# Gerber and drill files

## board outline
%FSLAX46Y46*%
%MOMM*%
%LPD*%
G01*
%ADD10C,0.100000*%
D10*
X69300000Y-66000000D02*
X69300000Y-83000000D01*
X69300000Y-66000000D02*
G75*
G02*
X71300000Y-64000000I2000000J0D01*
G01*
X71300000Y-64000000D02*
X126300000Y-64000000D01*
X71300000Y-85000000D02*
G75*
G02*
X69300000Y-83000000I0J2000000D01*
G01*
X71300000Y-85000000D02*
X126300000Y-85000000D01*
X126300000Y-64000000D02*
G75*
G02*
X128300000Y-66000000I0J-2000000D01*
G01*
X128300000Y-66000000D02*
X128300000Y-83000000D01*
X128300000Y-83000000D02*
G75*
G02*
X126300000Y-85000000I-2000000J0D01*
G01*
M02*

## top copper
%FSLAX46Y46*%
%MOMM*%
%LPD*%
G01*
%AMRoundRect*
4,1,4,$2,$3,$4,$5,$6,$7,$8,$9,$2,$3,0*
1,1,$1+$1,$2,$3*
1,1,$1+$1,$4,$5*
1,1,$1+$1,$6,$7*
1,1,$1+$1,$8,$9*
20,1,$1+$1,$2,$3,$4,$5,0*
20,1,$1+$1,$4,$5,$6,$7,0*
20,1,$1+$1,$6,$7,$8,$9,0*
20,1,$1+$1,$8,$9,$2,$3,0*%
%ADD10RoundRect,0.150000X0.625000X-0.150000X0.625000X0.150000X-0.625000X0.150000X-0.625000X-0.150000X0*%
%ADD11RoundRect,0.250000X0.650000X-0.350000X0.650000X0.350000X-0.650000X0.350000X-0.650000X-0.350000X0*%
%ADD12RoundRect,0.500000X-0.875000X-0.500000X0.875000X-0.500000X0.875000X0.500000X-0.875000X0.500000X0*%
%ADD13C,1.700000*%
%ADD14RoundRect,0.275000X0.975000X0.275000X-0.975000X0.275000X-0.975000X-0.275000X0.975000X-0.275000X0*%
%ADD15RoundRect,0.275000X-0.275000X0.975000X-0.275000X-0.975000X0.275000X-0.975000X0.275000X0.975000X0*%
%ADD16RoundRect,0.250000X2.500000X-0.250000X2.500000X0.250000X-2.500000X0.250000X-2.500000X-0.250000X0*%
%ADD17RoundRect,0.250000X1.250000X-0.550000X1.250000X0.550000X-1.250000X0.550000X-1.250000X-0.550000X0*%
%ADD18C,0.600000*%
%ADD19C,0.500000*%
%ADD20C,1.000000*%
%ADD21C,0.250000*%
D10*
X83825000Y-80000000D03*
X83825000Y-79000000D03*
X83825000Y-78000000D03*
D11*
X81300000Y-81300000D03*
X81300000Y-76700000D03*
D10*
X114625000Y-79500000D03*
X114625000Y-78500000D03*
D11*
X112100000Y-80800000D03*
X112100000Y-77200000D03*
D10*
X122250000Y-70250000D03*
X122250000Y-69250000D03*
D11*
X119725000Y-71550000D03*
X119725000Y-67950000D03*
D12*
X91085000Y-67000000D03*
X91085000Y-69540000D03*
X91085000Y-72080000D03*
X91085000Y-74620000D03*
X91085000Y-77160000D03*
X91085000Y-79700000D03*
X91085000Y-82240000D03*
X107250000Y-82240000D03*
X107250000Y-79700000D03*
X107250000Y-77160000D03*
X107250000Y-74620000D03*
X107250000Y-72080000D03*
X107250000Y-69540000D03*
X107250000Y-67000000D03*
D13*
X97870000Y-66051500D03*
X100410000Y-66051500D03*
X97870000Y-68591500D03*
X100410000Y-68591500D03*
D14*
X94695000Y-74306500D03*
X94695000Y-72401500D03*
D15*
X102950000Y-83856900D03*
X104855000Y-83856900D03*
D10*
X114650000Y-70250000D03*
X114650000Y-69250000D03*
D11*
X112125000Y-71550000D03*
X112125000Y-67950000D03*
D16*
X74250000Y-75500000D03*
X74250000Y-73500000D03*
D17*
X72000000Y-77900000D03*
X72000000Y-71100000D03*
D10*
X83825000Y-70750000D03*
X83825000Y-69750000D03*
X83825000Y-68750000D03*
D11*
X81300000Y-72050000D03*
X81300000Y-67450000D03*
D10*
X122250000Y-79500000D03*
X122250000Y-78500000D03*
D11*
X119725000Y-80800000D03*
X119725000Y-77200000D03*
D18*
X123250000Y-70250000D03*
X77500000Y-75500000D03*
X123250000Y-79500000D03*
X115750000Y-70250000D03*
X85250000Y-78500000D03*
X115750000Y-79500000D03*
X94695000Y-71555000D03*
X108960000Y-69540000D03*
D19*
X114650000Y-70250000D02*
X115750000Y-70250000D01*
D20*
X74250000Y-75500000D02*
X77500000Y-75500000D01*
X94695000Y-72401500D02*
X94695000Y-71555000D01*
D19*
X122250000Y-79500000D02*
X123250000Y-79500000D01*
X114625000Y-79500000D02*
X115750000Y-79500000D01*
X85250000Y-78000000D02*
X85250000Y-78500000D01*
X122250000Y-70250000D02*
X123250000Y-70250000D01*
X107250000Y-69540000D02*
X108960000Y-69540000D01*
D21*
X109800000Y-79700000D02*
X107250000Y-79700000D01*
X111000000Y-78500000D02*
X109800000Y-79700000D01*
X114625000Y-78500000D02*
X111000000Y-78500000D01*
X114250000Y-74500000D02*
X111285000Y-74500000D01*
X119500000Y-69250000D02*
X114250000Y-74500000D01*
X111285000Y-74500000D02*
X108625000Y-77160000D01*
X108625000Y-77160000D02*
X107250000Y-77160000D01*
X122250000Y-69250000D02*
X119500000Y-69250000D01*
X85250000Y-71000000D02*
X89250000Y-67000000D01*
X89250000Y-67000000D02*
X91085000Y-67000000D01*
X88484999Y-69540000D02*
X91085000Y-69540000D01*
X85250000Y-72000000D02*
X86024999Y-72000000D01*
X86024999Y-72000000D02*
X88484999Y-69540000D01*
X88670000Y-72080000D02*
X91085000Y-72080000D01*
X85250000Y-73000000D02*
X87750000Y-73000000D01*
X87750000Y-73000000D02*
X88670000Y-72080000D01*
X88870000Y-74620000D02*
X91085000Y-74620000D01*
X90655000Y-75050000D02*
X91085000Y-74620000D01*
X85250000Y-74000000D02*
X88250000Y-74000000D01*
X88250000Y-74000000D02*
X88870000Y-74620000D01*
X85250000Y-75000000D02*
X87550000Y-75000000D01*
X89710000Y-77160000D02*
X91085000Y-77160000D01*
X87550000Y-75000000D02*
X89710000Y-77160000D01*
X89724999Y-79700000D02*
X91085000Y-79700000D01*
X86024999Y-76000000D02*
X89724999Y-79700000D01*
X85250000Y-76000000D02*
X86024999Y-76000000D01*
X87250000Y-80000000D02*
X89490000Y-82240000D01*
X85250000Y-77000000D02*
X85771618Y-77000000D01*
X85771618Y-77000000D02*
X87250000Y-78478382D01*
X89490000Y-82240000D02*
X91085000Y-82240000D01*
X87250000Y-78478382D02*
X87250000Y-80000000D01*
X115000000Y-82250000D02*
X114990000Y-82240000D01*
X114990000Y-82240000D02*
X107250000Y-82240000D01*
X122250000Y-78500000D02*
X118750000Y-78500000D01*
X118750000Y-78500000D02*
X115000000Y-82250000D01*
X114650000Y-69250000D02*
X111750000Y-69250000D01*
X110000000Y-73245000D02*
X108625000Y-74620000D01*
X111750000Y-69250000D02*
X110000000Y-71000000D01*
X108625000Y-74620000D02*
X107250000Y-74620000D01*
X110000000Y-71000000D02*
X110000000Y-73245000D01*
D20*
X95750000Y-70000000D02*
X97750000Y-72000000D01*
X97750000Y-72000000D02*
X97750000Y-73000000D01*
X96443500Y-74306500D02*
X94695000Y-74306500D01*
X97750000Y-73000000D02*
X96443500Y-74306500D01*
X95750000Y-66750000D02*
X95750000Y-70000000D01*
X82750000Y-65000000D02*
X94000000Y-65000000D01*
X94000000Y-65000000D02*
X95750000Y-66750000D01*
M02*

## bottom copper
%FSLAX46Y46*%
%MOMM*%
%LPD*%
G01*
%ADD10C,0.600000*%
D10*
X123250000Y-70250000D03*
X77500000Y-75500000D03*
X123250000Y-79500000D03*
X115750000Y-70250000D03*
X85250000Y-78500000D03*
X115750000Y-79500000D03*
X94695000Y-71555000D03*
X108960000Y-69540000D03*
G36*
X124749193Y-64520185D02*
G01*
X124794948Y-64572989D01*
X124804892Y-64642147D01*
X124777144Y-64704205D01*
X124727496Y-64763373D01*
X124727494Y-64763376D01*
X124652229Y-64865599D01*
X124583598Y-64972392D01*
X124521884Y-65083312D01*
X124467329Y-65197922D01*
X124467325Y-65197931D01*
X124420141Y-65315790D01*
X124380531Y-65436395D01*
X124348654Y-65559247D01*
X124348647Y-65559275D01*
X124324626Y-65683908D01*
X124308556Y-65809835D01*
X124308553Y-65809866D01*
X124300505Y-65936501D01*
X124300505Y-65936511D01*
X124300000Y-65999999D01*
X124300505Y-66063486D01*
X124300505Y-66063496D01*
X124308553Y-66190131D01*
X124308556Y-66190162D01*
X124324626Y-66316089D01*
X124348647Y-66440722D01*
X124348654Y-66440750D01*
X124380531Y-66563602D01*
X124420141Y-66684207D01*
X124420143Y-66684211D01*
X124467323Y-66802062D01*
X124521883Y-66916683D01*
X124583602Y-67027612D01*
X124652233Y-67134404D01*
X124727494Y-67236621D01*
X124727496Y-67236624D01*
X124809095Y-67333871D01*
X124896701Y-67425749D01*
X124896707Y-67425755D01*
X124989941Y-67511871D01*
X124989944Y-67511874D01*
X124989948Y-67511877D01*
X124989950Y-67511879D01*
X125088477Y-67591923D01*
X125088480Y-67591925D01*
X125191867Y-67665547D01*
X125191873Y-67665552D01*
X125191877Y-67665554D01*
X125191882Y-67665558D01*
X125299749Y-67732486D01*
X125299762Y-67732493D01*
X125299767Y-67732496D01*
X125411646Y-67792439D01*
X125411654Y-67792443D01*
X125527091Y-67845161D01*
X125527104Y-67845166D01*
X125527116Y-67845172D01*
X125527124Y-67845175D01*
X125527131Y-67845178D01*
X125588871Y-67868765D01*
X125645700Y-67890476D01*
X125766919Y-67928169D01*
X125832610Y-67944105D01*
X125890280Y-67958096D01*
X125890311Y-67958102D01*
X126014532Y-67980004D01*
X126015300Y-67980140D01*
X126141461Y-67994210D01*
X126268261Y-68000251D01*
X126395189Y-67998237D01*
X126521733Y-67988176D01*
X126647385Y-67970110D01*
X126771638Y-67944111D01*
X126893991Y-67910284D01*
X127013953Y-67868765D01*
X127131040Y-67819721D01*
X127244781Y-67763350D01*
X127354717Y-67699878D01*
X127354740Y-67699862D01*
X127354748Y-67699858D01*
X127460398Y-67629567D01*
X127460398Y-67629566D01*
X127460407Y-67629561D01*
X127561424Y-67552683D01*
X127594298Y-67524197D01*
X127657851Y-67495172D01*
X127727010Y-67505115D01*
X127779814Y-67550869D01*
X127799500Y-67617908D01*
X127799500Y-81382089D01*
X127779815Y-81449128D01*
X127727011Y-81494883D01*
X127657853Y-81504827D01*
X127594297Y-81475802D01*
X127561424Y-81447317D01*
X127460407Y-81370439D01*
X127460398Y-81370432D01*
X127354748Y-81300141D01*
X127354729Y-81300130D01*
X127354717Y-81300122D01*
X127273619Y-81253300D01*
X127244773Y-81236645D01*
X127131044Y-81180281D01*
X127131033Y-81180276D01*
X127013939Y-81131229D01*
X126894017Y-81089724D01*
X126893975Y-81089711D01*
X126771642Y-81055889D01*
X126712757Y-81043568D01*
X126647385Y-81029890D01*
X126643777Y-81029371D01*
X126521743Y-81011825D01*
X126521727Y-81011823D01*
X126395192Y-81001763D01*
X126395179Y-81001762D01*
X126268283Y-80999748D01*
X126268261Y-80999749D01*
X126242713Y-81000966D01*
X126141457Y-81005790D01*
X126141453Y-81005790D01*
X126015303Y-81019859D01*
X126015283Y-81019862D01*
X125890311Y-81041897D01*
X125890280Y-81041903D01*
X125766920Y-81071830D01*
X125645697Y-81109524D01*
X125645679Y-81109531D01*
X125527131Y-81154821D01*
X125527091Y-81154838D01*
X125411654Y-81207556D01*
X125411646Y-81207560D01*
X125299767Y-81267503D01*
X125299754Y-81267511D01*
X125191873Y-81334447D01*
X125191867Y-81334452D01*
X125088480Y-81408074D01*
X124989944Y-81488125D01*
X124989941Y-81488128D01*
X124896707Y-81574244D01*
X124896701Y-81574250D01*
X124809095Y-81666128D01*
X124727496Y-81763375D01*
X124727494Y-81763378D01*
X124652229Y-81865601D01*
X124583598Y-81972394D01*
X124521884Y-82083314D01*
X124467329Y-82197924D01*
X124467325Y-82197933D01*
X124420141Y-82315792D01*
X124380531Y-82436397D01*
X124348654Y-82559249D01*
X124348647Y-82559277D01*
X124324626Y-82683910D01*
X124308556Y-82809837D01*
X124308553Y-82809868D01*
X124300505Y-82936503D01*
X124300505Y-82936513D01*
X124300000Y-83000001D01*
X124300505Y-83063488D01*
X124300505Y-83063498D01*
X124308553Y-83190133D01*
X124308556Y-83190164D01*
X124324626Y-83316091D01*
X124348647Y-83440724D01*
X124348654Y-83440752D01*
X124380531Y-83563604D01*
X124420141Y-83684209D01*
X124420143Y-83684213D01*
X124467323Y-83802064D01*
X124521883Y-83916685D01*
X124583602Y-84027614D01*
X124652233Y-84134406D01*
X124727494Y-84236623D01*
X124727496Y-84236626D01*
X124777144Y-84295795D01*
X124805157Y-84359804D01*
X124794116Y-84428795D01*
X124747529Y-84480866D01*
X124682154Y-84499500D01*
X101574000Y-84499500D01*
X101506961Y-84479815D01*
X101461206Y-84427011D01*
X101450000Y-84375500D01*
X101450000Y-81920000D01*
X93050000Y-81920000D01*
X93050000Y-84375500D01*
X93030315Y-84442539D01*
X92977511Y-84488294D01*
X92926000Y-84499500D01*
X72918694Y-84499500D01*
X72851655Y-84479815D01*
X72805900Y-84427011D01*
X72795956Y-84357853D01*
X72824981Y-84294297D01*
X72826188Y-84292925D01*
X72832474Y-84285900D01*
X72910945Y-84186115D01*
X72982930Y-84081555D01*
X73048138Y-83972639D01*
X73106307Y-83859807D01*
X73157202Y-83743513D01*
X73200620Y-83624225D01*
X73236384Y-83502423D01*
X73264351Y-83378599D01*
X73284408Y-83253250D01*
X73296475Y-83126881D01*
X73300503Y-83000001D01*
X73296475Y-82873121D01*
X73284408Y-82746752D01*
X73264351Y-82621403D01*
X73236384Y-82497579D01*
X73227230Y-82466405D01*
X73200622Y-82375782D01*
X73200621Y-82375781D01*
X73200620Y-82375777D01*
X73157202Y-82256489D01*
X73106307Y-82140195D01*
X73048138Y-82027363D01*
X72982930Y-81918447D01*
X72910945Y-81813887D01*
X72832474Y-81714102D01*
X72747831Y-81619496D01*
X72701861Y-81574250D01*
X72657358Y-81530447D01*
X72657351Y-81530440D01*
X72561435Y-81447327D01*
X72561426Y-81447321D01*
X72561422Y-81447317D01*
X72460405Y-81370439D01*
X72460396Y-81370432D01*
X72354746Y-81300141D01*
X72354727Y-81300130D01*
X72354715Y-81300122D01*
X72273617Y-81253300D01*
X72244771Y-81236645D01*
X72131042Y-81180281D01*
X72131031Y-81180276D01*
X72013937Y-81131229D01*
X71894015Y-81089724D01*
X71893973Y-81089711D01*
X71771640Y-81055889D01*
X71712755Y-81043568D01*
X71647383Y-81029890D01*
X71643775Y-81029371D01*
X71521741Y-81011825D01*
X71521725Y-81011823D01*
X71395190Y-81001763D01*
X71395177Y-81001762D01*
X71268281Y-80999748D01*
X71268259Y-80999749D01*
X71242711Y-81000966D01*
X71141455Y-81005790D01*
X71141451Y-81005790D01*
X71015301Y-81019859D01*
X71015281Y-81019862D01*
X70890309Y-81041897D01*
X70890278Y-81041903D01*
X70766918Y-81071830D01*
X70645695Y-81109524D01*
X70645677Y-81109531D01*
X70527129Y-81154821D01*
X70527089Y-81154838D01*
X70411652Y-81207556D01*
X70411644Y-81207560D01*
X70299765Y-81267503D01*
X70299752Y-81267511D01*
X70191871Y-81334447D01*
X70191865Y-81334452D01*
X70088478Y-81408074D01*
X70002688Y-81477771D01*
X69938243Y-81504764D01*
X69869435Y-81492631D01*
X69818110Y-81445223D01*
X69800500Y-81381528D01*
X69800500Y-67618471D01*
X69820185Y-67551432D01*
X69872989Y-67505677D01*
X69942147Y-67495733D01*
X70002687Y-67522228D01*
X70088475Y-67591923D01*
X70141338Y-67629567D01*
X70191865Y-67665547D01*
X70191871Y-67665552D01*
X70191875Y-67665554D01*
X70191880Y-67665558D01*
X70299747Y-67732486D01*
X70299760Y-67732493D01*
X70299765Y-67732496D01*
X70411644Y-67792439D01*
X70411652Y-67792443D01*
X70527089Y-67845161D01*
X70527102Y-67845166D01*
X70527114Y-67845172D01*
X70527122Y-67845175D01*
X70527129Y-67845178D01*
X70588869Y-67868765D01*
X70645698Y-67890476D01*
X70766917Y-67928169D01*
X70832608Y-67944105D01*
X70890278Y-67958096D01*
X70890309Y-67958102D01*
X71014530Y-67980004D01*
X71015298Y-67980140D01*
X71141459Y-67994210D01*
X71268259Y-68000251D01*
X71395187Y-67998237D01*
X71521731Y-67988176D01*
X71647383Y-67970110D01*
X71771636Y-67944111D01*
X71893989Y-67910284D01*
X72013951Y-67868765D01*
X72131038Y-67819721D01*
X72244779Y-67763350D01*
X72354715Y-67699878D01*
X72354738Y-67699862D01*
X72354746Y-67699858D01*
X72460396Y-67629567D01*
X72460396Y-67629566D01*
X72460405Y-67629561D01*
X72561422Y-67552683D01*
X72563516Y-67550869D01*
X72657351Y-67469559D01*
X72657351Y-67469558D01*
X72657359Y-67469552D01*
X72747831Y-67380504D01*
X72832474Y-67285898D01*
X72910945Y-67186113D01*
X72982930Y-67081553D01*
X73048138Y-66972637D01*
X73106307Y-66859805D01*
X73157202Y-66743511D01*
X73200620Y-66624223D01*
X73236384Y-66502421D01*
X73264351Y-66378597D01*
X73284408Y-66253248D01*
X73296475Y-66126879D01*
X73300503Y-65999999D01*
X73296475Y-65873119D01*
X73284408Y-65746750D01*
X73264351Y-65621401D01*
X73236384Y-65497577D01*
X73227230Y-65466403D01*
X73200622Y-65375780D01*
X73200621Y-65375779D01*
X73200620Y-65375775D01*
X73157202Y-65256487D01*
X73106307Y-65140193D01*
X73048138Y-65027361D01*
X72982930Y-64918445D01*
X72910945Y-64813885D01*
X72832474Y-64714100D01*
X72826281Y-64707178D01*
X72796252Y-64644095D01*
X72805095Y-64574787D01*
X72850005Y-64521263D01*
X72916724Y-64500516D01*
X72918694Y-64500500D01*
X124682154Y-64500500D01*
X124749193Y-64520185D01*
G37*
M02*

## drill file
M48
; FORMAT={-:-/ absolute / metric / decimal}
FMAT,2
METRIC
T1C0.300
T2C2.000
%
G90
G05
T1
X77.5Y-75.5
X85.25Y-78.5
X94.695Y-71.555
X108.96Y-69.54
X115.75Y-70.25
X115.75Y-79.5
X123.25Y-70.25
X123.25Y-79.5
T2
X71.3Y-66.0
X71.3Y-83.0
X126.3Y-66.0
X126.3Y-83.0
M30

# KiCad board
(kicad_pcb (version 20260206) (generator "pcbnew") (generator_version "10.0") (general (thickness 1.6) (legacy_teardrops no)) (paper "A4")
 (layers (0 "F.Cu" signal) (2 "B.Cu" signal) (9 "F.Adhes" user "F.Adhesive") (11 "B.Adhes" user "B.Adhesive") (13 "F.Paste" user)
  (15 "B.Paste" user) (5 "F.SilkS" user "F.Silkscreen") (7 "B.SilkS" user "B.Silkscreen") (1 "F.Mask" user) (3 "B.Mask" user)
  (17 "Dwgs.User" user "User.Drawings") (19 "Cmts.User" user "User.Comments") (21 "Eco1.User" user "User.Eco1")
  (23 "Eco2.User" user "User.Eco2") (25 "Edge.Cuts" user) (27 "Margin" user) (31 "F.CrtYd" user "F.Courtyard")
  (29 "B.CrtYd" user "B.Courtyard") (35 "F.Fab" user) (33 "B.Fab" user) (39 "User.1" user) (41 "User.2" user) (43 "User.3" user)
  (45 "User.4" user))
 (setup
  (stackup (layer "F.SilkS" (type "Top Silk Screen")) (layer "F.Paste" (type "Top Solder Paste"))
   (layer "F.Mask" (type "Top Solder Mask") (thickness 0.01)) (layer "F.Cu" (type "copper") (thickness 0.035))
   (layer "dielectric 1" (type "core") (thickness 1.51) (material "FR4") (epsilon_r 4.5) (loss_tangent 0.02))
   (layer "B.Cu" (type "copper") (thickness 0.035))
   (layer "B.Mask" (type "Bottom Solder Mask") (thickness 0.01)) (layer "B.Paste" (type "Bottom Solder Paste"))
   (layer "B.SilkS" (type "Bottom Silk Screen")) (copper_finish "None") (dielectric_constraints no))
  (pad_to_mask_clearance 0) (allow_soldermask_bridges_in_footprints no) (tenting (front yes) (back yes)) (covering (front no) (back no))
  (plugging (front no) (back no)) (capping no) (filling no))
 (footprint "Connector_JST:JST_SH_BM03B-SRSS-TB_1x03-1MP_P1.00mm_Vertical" (layer "F.Cu") (at 82.5 79 90)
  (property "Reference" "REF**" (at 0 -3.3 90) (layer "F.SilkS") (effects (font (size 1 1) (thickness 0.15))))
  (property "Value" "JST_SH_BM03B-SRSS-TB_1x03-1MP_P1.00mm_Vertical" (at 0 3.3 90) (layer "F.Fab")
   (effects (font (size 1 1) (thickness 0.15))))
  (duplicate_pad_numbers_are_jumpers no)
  (pad "1" smd roundrect (at -1 1.325 90) (size 0.6 1.55) (layers "F.Cu" "F.Mask" "F.Paste") (roundrect_rratio 0.25))
  (pad "2" smd roundrect (at 0 1.325 90) (size 0.6 1.55) (layers "F.Cu" "F.Mask" "F.Paste") (roundrect_rratio 0.25))
  (pad "3" smd roundrect (at 1 1.325 90) (size 0.6 1.55) (layers "F.Cu" "F.Mask" "F.Paste") (roundrect_rratio 0.25))
  (pad "MP" smd roundrect (at -2.3 -1.2 90) (size 1.2 1.8) (layers "F.Cu" "F.Mask" "F.Paste") (roundrect_rratio 0.208333))
  (pad "MP" smd roundrect (at 2.3 -1.2 90) (size 1.2 1.8) (layers "F.Cu" "F.Mask" "F.Paste") (roundrect_rratio 0.208333)))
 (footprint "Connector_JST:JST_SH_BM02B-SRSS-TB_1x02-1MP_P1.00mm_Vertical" (layer "F.Cu") (at 113.3 79 90)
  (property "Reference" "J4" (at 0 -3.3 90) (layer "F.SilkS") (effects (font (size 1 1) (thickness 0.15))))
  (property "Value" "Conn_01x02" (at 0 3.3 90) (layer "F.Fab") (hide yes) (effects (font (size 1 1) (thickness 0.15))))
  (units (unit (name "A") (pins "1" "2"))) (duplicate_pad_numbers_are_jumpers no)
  (pad "1" smd roundrect (at -0.5 1.325 90) (size 0.6 1.55) (layers "F.Cu" "F.Mask" "F.Paste") (roundrect_rratio 0.25) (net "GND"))
  (pad "2" smd roundrect (at 0.5 1.325 90) (size 0.6 1.55) (layers "F.Cu" "F.Mask" "F.Paste") (roundrect_rratio 0.25) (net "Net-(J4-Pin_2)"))
  (pad "MP" smd roundrect (at -1.8 -1.2 90) (size 1.2 1.8) (layers "F.Cu" "F.Mask" "F.Paste") (roundrect_rratio 0.208333))
  (pad "MP" smd roundrect (at 1.8 -1.2 90) (size 1.2 1.8) (layers "F.Cu" "F.Mask" "F.Paste") (roundrect_rratio 0.208333)))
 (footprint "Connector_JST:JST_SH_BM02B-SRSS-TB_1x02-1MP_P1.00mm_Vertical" (layer "F.Cu") (at 120.925 69.75 90)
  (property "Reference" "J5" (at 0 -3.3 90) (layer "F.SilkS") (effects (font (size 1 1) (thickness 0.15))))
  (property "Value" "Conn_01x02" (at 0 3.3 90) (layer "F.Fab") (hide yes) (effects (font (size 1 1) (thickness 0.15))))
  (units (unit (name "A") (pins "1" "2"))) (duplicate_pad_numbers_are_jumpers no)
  (pad "1" smd roundrect (at -0.5 1.325 90) (size 0.6 1.55) (layers "F.Cu" "F.Mask" "F.Paste") (roundrect_rratio 0.25) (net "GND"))
  (pad "2" smd roundrect (at 0.5 1.325 90) (size 0.6 1.55) (layers "F.Cu" "F.Mask" "F.Paste") (roundrect_rratio 0.25) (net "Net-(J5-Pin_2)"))
  (pad "MP" smd roundrect (at -1.8 -1.2 90) (size 1.2 1.8) (layers "F.Cu" "F.Mask" "F.Paste") (roundrect_rratio 0.208333))
  (pad "MP" smd roundrect (at 1.8 -1.2 90) (size 1.2 1.8) (layers "F.Cu" "F.Mask" "F.Paste") (roundrect_rratio 0.208333)))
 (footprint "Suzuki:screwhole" (layer "F.Cu") (at 126.300001 65.999999)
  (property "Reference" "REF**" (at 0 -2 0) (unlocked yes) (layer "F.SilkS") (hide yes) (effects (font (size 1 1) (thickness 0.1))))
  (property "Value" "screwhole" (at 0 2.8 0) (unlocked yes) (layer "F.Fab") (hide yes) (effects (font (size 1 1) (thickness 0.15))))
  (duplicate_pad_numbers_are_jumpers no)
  (pad "" np_thru_hole circle (at 0 0) (size 2 2) (drill 2) (layers "*.Cu" "*.Mask"))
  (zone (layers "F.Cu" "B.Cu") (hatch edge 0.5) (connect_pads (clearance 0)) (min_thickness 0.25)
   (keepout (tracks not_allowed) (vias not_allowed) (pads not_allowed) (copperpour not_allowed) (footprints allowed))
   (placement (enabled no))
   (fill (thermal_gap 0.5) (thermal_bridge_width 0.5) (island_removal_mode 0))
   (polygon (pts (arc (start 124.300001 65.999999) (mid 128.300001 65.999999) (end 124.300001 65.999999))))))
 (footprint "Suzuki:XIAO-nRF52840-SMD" (layer "F.Cu") (at 90.25 85.12)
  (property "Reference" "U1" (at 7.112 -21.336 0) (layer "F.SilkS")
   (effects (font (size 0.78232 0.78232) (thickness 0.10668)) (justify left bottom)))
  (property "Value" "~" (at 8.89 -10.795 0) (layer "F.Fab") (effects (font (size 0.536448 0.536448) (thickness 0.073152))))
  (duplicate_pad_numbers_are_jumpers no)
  (pad "1" smd roundrect (at 0.835 -18.12) (size 2.75 2) (layers "F.Cu" "F.Mask" "F.Paste") (roundrect_rratio 0.25) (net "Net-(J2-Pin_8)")
   (solder_mask_margin 0.0508) (thermal_bridge_angle 45))
  (pad "2" smd roundrect (at 0.835 -15.58) (size 2.75 2) (layers "F.Cu" "F.Mask" "F.Paste") (roundrect_rratio 0.25) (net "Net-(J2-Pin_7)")
   (solder_mask_margin 0.0508) (thermal_bridge_angle 45))
  (pad "3" smd roundrect (at 0.835 -13.04) (size 2.75 2) (layers "F.Cu" "F.Mask" "F.Paste") (roundrect_rratio 0.25) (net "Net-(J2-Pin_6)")
   (solder_mask_margin 0.0508) (thermal_bridge_angle 45))
  (pad "4" smd roundrect (at 0.835 -10.5) (size 2.75 2) (layers "F.Cu" "F.Mask" "F.Paste") (roundrect_rratio 0.25) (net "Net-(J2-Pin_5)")
   (solder_mask_margin 0.0508) (thermal_bridge_angle 45))
  (pad "5" smd roundrect (at 0.835 -7.96) (size 2.75 2) (layers "F.Cu" "F.Mask" "F.Paste") (roundrect_rratio 0.25) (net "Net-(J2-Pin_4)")
   (solder_mask_margin 0.0508) (thermal_bridge_angle 45))
  (pad "6" smd roundrect (at 0.835 -5.42) (size 2.75 2) (layers "F.Cu" "F.Mask" "F.Paste") (roundrect_rratio 0.25) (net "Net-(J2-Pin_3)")
   (solder_mask_margin 0.0508) (thermal_bridge_angle 45))
  (pad "7" smd roundrect (at 0.835 -2.88) (size 2.75 2) (layers "F.Cu" "F.Mask" "F.Paste") (roundrect_rratio 0.25) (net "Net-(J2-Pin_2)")
   (solder_mask_margin 0.0508) (thermal_bridge_angle 45))
  (pad "8" smd roundrect (at 17 -2.88) (size 2.75 2) (layers "F.Cu" "F.Mask" "F.Paste") (roundrect_rratio 0.25) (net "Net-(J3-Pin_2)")
   (solder_mask_margin 0.0508) (thermal_bridge_angle 45))
  (pad "9" smd roundrect (at 17 -5.42) (size 2.75 2) (layers "F.Cu" "F.Mask" "F.Paste") (roundrect_rratio 0.25) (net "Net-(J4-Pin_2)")
   (solder_mask_margin 0.0508) (thermal_bridge_angle 45))
  (pad "10" smd roundrect (at 17 -7.96) (size 2.75 2) (layers "F.Cu" "F.Mask" "F.Paste") (roundrect_rratio 0.25) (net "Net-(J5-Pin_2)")
   (solder_mask_margin 0.0508) (thermal_bridge_angle 45))
  (pad "11" smd roundrect (at 17 -10.5) (size 2.75 2) (layers "F.Cu" "F.Mask" "F.Paste") (roundrect_rratio 0.25) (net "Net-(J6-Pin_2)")
   (solder_mask_margin 0.0508) (thermal_bridge_angle 45))
  (pad "12" smd roundrect (at 17 -13.04) (size 2.75 2) (layers "F.Cu" "F.Mask" "F.Paste") (roundrect_rratio 0.25)
   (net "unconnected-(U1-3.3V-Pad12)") (solder_mask_margin 0.0508) (thermal_bridge_angle 45))
  (pad "13" smd roundrect (at 17 -15.58) (size 2.75 2) (layers "F.Cu" "F.Mask" "F.Paste") (roundrect_rratio 0.25) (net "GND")
   (solder_mask_margin 0.0508) (thermal_bridge_angle 45))
  (pad "14" smd roundrect (at 17 -18.12) (size 2.75 2) (layers "F.Cu" "F.Mask" "F.Paste") (roundrect_rratio 0.25)
   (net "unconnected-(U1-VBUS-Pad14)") (solder_mask_margin 0.0508) (thermal_bridge_angle 45))
  (pad "15" smd circle (at 7.62 -19.0685) (size 1.7 1.7) (layers "F.Cu" "F.Mask" "F.Paste"))
  (pad "16" smd circle (at 10.16 -19.0685) (size 1.7 1.7) (layers "F.Cu" "F.Mask" "F.Paste"))
  (pad "17" smd circle (at 7.62 -16.5285) (size 1.7 1.7) (layers "F.Cu" "F.Mask" "F.Paste"))
  (pad "18" smd circle (at 10.16 -16.5285) (size 1.7 1.7) (layers "F.Cu" "F.Mask" "F.Paste"))
  (pad "19" smd roundrect (at 4.445 -10.8135 180) (size 2.5 1.1) (layers "F.Cu" "F.Mask" "F.Paste") (roundrect_rratio 0.25)
   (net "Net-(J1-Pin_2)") (thermal_bridge_angle 45))
  (pad "20" smd roundrect (at 4.445 -12.7185 180) (size 2.5 1.1) (layers "F.Cu" "F.Mask" "F.Paste") (roundrect_rratio 0.25) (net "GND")
   (thermal_bridge_angle 45))
  (pad "21" smd roundrect (at 12.7 -1.2631 270) (size 2.5 1.1) (layers "F.Cu" "F.Mask" "F.Paste") (roundrect_rratio 0.25)
   (thermal_bridge_angle 45))
  (pad "22" smd roundrect (at 14.605 -1.2631 270) (size 2.5 1.1) (layers "F.Cu" "F.Mask" "F.Paste") (roundrect_rratio 0.25)
   (thermal_bridge_angle 45))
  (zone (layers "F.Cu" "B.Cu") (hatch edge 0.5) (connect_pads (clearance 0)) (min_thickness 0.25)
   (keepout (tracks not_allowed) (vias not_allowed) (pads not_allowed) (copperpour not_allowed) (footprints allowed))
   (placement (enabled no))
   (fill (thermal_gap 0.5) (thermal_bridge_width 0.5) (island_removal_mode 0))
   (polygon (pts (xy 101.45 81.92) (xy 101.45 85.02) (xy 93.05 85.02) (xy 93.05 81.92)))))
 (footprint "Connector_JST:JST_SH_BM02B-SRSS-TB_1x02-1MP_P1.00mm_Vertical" (layer "F.Cu") (at 113.325 69.75 90)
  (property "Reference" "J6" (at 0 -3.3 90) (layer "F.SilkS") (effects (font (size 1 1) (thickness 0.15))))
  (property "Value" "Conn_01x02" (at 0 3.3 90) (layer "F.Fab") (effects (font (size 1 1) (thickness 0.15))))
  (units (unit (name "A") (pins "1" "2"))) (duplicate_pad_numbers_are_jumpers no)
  (pad "1" smd roundrect (at -0.5 1.325 90) (size 0.6 1.55) (layers "F.Cu" "F.Mask" "F.Paste") (roundrect_rratio 0.25) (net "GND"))
  (pad "2" smd roundrect (at 0.5 1.325 90) (size 0.6 1.55) (layers "F.Cu" "F.Mask" "F.Paste") (roundrect_rratio 0.25) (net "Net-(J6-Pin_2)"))
  (pad "MP" smd roundrect (at -1.8 -1.2 90) (size 1.2 1.8) (layers "F.Cu" "F.Mask" "F.Paste") (roundrect_rratio 0.208333))
  (pad "MP" smd roundrect (at 1.8 -1.2 90) (size 1.2 1.8) (layers "F.Cu" "F.Mask" "F.Paste") (roundrect_rratio 0.208333)))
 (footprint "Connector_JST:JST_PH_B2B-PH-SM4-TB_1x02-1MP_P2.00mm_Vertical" (layer "F.Cu") (at 73.75 74.5 90)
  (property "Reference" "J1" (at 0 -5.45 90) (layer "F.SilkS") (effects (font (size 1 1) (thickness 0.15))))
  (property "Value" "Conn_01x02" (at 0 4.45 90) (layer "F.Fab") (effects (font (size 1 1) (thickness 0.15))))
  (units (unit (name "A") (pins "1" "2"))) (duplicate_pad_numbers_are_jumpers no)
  (pad "1" smd roundrect (at -1 0.5 90) (size 1 5.5) (layers "F.Cu" "F.Mask" "F.Paste") (roundrect_rratio 0.25) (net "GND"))
  (pad "2" smd roundrect (at 1 0.5 90) (size 1 5.5) (layers "F.Cu" "F.Mask" "F.Paste") (roundrect_rratio 0.25) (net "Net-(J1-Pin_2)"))
  (pad "MP" smd roundrect (at -3.4 -1.75 90) (size 1.6 3) (layers "F.Cu" "F.Mask" "F.Paste") (roundrect_rratio 0.15625))
  (pad "MP" smd roundrect (at 3.4 -1.75 90) (size 1.6 3) (layers "F.Cu" "F.Mask" "F.Paste") (roundrect_rratio 0.15625)))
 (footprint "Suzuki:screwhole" (layer "F.Cu") (at 71.299999 83.000001)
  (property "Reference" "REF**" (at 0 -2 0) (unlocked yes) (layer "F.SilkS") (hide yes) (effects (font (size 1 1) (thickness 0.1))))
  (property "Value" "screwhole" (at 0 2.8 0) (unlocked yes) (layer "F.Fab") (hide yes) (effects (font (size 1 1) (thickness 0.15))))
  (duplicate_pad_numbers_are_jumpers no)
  (pad "" np_thru_hole circle (at 0 0) (size 2 2) (drill 2) (layers "*.Cu" "*.Mask"))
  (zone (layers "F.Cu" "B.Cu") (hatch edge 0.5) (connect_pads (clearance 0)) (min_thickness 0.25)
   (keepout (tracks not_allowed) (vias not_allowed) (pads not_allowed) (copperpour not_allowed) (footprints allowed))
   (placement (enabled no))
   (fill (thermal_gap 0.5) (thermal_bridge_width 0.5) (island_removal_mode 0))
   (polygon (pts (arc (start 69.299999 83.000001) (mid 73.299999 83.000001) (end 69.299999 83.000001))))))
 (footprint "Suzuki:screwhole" (layer "F.Cu") (at 126.300001 83.000001)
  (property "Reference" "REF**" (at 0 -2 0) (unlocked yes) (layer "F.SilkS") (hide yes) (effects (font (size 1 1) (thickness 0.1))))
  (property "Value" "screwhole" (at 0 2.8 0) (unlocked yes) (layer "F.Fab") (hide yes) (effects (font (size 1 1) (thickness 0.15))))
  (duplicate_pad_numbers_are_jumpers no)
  (pad "" np_thru_hole circle (at 0 0) (size 2 2) (drill 2) (layers "*.Cu" "*.Mask"))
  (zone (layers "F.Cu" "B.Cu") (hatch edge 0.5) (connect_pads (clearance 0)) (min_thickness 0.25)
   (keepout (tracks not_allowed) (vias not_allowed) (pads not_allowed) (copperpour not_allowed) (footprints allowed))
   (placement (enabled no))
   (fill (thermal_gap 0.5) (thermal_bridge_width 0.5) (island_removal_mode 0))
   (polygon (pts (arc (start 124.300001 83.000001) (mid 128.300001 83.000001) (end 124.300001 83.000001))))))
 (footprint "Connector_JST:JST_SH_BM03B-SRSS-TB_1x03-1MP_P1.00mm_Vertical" (layer "F.Cu") (at 82.5 69.75 90)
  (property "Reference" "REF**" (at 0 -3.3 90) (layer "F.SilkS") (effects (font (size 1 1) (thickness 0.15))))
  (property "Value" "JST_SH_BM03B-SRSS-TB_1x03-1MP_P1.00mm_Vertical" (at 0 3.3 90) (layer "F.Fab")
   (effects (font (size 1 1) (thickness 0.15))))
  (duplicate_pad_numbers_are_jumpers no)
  (pad "1" smd roundrect (at -1 1.325 90) (size 0.6 1.55) (layers "F.Cu" "F.Mask" "F.Paste") (roundrect_rratio 0.25))
  (pad "2" smd roundrect (at 0 1.325 90) (size 0.6 1.55) (layers "F.Cu" "F.Mask" "F.Paste") (roundrect_rratio 0.25))
  (pad "3" smd roundrect (at 1 1.325 90) (size 0.6 1.55) (layers "F.Cu" "F.Mask" "F.Paste") (roundrect_rratio 0.25))
  (pad "MP" smd roundrect (at -2.3 -1.2 90) (size 1.2 1.8) (layers "F.Cu" "F.Mask" "F.Paste") (roundrect_rratio 0.208333))
  (pad "MP" smd roundrect (at 2.3 -1.2 90) (size 1.2 1.8) (layers "F.Cu" "F.Mask" "F.Paste") (roundrect_rratio 0.208333)))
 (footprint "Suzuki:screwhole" (layer "F.Cu") (at 71.299999 65.999999)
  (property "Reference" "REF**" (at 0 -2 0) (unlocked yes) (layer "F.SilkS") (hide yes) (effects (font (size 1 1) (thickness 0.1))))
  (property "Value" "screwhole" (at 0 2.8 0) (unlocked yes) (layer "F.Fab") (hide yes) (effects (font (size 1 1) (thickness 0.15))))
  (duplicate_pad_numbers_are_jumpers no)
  (pad "" np_thru_hole circle (at 0 0) (size 2 2) (drill 2) (layers "*.Cu" "*.Mask"))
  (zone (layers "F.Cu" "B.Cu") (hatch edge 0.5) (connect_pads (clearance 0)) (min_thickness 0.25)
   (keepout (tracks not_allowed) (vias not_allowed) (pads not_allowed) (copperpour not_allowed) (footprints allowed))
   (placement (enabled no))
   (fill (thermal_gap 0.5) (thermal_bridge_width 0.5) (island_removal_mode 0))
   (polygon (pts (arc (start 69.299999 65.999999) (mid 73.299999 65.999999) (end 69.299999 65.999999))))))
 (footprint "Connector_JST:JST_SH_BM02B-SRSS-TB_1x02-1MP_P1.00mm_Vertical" (layer "F.Cu") (at 120.925 79 90)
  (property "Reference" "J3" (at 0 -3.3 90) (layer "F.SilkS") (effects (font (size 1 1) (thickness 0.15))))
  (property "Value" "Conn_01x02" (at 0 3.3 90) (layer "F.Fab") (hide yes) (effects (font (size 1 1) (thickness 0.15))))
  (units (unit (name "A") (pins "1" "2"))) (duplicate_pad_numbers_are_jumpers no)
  (pad "1" smd roundrect (at -0.5 1.325 90) (size 0.6 1.55) (layers "F.Cu" "F.Mask" "F.Paste") (roundrect_rratio 0.25) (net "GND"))
  (pad "2" smd roundrect (at 0.5 1.325 90) (size 0.6 1.55) (layers "F.Cu" "F.Mask" "F.Paste") (roundrect_rratio 0.25) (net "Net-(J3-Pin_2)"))
  (pad "MP" smd roundrect (at -1.8 -1.2 90) (size 1.2 1.8) (layers "F.Cu" "F.Mask" "F.Paste") (roundrect_rratio 0.208333))
  (pad "MP" smd roundrect (at 1.8 -1.2 90) (size 1.2 1.8) (layers "F.Cu" "F.Mask" "F.Paste") (roundrect_rratio 0.208333)))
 (gr_line (start 69.3 66) (end 69.3 83) (stroke (width 0.1) (type solid)) (layer "Edge.Cuts"))
 (gr_arc (start 69.3 66) (mid 69.885786 64.585786) (end 71.3 64) (stroke (width 0.1) (type default)) (layer "Edge.Cuts"))
 (gr_line (start 71.3 64) (end 126.3 64) (stroke (width 0.1) (type solid)) (layer "Edge.Cuts"))
 (gr_arc (start 71.3 85) (mid 69.885786 84.414214) (end 69.3 83) (stroke (width 0.1) (type default)) (layer "Edge.Cuts"))
 (gr_line (start 71.3 85) (end 126.3 85) (stroke (width 0.1) (type solid)) (layer "Edge.Cuts"))
 (gr_arc (start 126.3 64) (mid 127.714214 64.585786) (end 128.3 66) (stroke (width 0.1) (type default)) (layer "Edge.Cuts"))
 (gr_line (start 128.3 66) (end 128.3 83) (stroke (width 0.1) (type solid)) (layer "Edge.Cuts"))
 (gr_arc (start 128.3 83) (mid 127.714214 84.414214) (end 126.3 85) (stroke (width 0.1) (type default)) (layer "Edge.Cuts"))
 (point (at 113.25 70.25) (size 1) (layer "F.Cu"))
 (segment (start 114.65 70.25) (end 115.75 70.25) (width 0.5) (layer "F.Cu") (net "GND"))
 (segment (start 74.25 75.5) (end 77.5 75.5) (width 1) (layer "F.Cu") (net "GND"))
 (segment (start 94.695 72.4015) (end 94.695 71.555) (width 1) (layer "F.Cu") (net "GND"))
 (segment (start 122.25 79.5) (end 123.25 79.5) (width 0.5) (layer "F.Cu") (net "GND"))
 (segment (start 114.625 79.5) (end 115.75 79.5) (width 0.5) (layer "F.Cu") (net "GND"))
 (segment (start 85.25 78) (end 85.25 78.5) (width 0.5) (layer "F.Cu") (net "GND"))
 (segment (start 122.25 70.25) (end 123.25 70.25) (width 0.5) (layer "F.Cu") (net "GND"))
 (segment (start 107.25 69.54) (end 108.96 69.54) (width 0.5) (layer "F.Cu") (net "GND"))
 (via (at 123.25 70.25) (size 0.6) (drill 0.3) (layers "F.Cu" "B.Cu") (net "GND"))
 (via (at 77.5 75.5) (size 0.6) (drill 0.3) (layers "F.Cu" "B.Cu") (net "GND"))
 (via (at 123.25 79.5) (size 0.6) (drill 0.3) (layers "F.Cu" "B.Cu") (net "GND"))
 (via (at 115.75 70.25) (size 0.6) (drill 0.3) (layers "F.Cu" "B.Cu") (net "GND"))
 (via (at 85.25 78.5) (size 0.6) (drill 0.3) (layers "F.Cu" "B.Cu") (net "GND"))
 (via (at 115.75 79.5) (size 0.6) (drill 0.3) (layers "F.Cu" "B.Cu") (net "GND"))
 (via (at 94.695 71.555) (size 0.6) (drill 0.3) (layers "F.Cu" "B.Cu") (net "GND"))
 (via (at 108.96 69.54) (size 0.6) (drill 0.3) (layers "F.Cu" "B.Cu") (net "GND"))
 (segment (start 109.8 79.7) (end 107.25 79.7) (width 0.25) (layer "F.Cu") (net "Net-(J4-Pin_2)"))
 (segment (start 111 78.5) (end 109.8 79.7) (width 0.25) (layer "F.Cu") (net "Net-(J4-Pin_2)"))
 (segment (start 114.625 78.5) (end 111 78.5) (width 0.25) (layer "F.Cu") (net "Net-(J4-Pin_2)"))
 (segment (start 114.25 74.5) (end 111.285 74.5) (width 0.25) (layer "F.Cu") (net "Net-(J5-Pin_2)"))
 (segment (start 119.5 69.25) (end 114.25 74.5) (width 0.25) (layer "F.Cu") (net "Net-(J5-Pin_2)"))
 (segment (start 111.285 74.5) (end 108.625 77.16) (width 0.25) (layer "F.Cu") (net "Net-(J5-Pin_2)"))
 (segment (start 108.625 77.16) (end 107.25 77.16) (width 0.25) (layer "F.Cu") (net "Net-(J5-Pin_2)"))
 (segment (start 122.25 69.25) (end 119.5 69.25) (width 0.25) (layer "F.Cu") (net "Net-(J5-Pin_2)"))
 (segment (start 85.25 71) (end 89.25 67) (width 0.25) (layer "F.Cu") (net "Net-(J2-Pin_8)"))
 (segment (start 89.25 67) (end 91.085 67) (width 0.25) (layer "F.Cu") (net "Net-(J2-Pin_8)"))
 (segment (start 88.484999 69.54) (end 91.085 69.54) (width 0.25) (layer "F.Cu") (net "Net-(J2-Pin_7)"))
 (segment (start 85.25 72) (end 86.024999 72) (width 0.25) (layer "F.Cu") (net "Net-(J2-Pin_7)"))
 (segment (start 86.024999 72) (end 88.484999 69.54) (width 0.25) (layer "F.Cu") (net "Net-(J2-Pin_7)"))
 (segment (start 88.67 72.08) (end 91.085 72.08) (width 0.25) (layer "F.Cu") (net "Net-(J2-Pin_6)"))
 (segment (start 85.25 73) (end 87.75 73) (width 0.25) (layer "F.Cu") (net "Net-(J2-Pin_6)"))
 (segment (start 87.75 73) (end 88.67 72.08) (width 0.25) (layer "F.Cu") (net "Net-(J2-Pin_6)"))
 (segment (start 88.87 74.62) (end 91.085 74.62) (width 0.25) (layer "F.Cu") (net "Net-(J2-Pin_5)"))
 (segment (start 90.655 75.05) (end 91.085 74.62) (width 0.25) (layer "F.Cu") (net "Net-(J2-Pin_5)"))
 (segment (start 85.25 74) (end 88.25 74) (width 0.25) (layer "F.Cu") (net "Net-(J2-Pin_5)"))
 (segment (start 88.25 74) (end 88.87 74.62) (width 0.25) (layer "F.Cu") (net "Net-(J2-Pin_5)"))
 (segment (start 85.25 75) (end 87.55 75) (width 0.25) (layer "F.Cu") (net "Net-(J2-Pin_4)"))
 (segment (start 89.71 77.16) (end 91.085 77.16) (width 0.25) (layer "F.Cu") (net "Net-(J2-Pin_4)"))
 (segment (start 87.55 75) (end 89.71 77.16) (width 0.25) (layer "F.Cu") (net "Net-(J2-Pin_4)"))
 (segment (start 89.724999 79.7) (end 91.085 79.7) (width 0.25) (layer "F.Cu") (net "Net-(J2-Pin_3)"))
 (segment (start 86.024999 76) (end 89.724999 79.7) (width 0.25) (layer "F.Cu") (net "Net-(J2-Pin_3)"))
 (segment (start 85.25 76) (end 86.024999 76) (width 0.25) (layer "F.Cu") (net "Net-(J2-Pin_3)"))
 (segment (start 87.25 80) (end 89.49 82.24) (width 0.25) (layer "F.Cu") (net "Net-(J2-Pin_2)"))
 (segment (start 85.25 77) (end 85.771618 77) (width 0.25) (layer "F.Cu") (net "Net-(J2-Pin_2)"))
 (segment (start 85.771618 77) (end 87.25 78.478382) (width 0.25) (layer "F.Cu") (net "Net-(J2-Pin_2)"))
 (segment (start 89.49 82.24) (end 91.085 82.24) (width 0.25) (layer "F.Cu") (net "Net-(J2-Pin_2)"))
 (segment (start 87.25 78.478382) (end 87.25 80) (width 0.25) (layer "F.Cu") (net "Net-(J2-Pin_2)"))
 (segment (start 115 82.25) (end 114.99 82.24) (width 0.25) (layer "F.Cu") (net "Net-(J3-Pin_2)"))
 (segment (start 114.99 82.24) (end 107.25 82.24) (width 0.25) (layer "F.Cu") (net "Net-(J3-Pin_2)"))
 (segment (start 122.25 78.5) (end 118.75 78.5) (width 0.25) (layer "F.Cu") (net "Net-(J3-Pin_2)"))
 (segment (start 118.75 78.5) (end 115 82.25) (width 0.25) (layer "F.Cu") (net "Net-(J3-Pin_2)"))
 (segment (start 114.65 69.25) (end 111.75 69.25) (width 0.25) (layer "F.Cu") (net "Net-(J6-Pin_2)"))
 (segment (start 110 73.245) (end 108.625 74.62) (width 0.25) (layer "F.Cu") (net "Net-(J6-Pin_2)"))
 (segment (start 111.75 69.25) (end 110 71) (width 0.25) (layer "F.Cu") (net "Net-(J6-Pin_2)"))
 (segment (start 108.625 74.62) (end 107.25 74.62) (width 0.25) (layer "F.Cu") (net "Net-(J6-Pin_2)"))
 (segment (start 110 71) (end 110 73.245) (width 0.25) (layer "F.Cu") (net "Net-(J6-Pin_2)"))
 (segment (start 95.75 70) (end 97.75 72) (width 1) (layer "F.Cu") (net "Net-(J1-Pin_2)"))
 (segment (start 97.75 72) (end 97.75 73) (width 1) (layer "F.Cu") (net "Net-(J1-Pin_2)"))
 (segment (start 96.4435 74.3065) (end 94.695 74.3065) (width 1) (layer "F.Cu") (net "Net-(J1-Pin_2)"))
 (segment (start 97.75 73) (end 96.4435 74.3065) (width 1) (layer "F.Cu") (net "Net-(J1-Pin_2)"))
 (segment (start 95.75 66.75) (end 95.75 70) (width 1) (layer "F.Cu") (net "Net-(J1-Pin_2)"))
 (segment (start 82.75 65) (end 94 65) (width 1) (layer "F.Cu") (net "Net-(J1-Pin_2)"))
 (segment (start 94 65) (end 95.75 66.75) (width 1) (layer "F.Cu") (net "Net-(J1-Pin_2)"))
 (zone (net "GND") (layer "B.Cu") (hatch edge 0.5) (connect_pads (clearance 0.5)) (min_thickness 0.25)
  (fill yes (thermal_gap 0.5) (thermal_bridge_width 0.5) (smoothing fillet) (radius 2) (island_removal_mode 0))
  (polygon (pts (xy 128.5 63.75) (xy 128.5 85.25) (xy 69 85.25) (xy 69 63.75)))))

